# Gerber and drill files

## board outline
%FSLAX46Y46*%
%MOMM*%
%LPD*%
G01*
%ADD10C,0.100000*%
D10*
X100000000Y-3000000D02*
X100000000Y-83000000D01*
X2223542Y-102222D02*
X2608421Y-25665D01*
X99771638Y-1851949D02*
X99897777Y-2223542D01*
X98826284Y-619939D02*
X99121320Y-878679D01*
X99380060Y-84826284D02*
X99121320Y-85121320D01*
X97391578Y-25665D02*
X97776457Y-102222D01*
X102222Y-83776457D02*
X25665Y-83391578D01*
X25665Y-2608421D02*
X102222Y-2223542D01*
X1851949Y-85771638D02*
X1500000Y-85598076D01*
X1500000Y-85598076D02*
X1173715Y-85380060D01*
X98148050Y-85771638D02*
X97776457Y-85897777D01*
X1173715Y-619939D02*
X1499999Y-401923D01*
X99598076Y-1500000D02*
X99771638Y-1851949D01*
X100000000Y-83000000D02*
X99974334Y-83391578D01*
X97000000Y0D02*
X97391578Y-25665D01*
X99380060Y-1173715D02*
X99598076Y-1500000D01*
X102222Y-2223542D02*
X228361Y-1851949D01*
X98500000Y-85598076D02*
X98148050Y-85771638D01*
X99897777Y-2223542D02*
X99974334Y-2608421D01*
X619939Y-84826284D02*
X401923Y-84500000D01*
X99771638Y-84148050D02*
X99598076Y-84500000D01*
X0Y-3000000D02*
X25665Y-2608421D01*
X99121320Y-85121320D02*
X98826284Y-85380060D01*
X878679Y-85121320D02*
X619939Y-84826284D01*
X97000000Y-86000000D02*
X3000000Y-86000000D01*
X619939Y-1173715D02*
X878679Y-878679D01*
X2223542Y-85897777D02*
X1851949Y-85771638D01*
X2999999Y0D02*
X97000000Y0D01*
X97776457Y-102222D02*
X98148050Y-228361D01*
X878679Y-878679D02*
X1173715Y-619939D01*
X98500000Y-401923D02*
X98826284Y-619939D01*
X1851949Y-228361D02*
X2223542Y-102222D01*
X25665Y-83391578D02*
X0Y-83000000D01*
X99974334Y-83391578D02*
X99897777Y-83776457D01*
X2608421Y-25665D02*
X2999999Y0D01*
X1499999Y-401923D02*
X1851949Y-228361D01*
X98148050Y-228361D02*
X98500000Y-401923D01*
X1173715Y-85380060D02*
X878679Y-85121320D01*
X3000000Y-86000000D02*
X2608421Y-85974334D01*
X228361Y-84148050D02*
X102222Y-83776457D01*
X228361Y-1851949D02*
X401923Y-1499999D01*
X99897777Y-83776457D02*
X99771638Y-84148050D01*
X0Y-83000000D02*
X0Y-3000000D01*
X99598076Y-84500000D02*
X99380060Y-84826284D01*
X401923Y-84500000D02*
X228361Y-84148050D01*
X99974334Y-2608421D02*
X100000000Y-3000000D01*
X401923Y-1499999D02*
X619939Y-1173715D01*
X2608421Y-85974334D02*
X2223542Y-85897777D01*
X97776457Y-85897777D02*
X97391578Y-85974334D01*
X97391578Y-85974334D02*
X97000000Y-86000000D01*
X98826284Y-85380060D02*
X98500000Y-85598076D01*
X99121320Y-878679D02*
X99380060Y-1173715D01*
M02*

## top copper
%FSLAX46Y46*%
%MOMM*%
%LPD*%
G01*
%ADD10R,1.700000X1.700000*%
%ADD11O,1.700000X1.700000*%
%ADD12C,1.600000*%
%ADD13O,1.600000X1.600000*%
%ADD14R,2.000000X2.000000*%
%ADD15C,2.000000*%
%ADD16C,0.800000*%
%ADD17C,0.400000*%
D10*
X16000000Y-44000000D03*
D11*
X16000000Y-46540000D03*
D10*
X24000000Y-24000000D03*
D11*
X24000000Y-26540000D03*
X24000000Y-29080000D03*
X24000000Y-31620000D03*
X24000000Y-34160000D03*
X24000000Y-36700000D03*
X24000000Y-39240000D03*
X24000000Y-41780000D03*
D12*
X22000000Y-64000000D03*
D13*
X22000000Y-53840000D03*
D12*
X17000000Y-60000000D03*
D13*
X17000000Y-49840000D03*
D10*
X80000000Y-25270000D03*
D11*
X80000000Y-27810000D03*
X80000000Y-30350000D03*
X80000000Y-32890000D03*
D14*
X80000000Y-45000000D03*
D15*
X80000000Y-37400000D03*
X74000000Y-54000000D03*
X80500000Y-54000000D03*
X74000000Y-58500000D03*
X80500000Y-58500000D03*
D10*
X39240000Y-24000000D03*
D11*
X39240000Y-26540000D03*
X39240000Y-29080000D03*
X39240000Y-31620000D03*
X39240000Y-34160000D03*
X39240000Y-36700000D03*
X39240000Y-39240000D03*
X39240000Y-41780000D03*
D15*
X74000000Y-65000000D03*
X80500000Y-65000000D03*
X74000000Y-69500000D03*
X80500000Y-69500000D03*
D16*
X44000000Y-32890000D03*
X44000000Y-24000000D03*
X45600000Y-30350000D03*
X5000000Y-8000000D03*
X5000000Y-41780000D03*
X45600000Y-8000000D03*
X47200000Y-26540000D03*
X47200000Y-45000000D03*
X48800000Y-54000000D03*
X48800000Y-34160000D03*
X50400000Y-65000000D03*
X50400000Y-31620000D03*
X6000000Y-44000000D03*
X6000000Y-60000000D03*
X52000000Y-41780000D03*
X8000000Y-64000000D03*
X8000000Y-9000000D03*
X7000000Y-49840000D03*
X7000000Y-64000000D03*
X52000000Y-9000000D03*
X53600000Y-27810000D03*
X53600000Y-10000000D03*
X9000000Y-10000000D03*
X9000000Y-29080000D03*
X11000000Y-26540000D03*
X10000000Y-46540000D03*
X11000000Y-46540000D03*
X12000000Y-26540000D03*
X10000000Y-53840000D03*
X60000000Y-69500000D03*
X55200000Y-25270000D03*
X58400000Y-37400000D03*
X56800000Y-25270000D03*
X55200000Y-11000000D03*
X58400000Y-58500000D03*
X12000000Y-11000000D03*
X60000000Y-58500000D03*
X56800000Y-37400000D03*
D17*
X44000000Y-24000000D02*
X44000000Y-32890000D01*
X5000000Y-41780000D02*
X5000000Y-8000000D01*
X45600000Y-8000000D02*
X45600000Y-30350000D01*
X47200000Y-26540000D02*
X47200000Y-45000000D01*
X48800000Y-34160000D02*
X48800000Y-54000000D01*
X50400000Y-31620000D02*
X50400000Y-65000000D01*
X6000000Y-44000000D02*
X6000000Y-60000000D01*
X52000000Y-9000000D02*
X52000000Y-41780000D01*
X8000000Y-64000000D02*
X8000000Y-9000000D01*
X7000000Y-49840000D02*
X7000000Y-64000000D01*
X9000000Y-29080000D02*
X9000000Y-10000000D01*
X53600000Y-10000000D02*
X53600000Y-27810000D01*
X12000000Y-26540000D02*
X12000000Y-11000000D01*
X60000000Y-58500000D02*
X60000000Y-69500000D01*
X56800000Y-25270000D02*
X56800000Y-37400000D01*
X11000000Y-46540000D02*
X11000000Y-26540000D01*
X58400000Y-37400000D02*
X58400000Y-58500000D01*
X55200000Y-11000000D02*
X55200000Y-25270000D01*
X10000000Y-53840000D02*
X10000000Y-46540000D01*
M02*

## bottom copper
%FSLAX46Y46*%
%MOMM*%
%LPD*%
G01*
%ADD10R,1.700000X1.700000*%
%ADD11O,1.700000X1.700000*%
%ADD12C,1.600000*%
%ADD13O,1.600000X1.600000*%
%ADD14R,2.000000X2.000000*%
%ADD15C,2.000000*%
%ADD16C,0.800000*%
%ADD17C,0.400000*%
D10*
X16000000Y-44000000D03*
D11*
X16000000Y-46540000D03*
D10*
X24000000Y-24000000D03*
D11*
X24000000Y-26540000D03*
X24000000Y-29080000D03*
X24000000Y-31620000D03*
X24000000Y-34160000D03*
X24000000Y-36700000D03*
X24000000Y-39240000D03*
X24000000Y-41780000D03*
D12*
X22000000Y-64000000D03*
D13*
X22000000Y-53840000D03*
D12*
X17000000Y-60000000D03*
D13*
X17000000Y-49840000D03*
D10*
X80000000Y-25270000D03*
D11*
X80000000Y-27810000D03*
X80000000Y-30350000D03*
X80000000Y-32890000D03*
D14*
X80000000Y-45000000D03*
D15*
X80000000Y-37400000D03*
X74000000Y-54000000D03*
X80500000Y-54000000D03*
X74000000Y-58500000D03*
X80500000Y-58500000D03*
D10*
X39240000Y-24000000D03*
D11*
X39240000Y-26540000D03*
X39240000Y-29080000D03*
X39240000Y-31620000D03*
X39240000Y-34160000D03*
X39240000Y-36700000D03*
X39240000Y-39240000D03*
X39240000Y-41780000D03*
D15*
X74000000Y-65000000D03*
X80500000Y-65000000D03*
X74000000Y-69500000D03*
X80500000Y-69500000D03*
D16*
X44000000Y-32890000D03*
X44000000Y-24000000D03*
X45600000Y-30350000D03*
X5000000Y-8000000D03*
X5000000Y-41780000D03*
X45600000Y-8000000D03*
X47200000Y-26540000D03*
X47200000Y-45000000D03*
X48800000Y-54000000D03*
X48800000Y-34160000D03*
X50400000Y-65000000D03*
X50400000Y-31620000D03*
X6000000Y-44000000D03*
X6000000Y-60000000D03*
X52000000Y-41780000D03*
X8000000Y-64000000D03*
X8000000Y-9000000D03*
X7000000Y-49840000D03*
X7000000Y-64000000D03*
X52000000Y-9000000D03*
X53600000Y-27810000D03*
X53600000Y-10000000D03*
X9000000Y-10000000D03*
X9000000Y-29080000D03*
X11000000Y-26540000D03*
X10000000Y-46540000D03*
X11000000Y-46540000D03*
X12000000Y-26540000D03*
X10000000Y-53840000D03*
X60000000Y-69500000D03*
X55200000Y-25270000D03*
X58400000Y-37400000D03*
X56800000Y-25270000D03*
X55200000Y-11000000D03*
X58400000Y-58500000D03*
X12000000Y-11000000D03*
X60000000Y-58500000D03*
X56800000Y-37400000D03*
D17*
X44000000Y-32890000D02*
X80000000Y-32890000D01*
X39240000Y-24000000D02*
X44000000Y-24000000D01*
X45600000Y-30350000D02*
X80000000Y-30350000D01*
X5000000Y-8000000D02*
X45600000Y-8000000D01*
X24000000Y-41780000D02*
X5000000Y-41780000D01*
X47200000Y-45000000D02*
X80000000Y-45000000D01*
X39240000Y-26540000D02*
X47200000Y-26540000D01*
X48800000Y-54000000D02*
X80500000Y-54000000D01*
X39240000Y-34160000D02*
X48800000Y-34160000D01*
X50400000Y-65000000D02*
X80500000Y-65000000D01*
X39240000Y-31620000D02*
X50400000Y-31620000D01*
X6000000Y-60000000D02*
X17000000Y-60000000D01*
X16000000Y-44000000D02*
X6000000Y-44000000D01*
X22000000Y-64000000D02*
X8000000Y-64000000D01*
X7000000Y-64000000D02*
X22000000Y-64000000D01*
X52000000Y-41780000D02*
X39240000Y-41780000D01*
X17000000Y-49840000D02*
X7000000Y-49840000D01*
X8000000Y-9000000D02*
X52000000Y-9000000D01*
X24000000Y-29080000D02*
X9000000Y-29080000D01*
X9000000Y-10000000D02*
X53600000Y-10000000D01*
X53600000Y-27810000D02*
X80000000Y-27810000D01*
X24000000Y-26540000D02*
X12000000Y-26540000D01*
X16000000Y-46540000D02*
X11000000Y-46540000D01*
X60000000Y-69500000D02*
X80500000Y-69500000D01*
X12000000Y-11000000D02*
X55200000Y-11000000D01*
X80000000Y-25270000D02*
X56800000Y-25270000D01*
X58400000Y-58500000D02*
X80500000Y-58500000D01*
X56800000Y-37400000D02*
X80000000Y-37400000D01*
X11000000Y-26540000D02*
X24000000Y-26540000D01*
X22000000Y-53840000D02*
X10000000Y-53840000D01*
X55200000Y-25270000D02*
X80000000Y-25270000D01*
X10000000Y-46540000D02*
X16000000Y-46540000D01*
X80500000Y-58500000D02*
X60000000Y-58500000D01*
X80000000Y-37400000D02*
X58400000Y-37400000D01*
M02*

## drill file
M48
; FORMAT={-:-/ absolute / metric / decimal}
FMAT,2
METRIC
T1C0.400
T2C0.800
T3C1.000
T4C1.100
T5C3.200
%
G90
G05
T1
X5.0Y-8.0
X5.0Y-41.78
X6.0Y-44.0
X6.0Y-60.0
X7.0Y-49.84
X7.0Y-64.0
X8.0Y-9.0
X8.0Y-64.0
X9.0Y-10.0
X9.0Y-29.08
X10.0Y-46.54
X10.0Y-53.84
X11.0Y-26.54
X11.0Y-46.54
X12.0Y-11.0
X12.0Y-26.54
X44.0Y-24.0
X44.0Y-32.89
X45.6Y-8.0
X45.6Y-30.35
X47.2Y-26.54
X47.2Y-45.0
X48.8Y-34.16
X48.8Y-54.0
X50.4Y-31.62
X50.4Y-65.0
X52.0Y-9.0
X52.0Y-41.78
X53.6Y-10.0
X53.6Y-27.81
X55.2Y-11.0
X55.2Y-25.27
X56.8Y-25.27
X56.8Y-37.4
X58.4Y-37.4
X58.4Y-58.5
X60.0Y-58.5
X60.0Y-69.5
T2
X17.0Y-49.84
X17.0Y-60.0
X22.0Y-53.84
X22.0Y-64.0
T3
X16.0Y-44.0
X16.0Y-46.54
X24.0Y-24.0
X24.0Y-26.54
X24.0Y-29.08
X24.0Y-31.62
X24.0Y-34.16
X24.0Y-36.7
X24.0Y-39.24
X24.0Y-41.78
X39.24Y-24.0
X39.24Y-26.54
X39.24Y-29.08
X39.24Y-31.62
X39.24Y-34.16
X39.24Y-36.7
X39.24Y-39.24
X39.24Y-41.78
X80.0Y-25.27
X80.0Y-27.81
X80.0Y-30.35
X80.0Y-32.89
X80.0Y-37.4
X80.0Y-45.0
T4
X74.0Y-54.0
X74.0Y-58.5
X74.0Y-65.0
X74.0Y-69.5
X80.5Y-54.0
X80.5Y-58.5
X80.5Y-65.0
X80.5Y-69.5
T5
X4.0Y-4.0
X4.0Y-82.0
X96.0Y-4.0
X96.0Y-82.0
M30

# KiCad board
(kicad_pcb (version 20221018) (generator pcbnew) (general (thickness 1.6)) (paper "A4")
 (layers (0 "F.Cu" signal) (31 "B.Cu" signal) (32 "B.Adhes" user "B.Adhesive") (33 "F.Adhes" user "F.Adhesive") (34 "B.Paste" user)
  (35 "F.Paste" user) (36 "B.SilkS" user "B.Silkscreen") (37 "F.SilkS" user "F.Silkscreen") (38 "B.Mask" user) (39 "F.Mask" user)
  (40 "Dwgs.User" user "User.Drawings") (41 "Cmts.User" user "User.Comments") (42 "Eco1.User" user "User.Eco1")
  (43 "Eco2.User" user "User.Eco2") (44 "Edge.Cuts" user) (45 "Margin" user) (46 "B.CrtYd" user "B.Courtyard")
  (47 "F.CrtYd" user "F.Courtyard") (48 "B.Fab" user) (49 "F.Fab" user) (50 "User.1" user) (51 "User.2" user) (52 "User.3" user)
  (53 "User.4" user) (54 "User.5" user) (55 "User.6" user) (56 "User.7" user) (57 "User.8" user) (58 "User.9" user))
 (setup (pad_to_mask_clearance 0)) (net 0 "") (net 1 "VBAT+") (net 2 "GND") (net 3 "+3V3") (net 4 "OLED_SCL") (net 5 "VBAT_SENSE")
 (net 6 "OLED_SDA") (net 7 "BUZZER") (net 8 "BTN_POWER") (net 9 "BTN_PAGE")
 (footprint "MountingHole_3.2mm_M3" (layer "F.Cu") (at 96 4)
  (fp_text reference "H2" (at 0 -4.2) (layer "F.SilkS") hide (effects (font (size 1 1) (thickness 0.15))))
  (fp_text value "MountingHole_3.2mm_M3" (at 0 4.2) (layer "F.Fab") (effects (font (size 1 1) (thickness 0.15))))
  (pad "" np_thru_hole circle (at 0 0) (size 3.2 3.2) (drill 3.2) (layers "*.Cu" "*.Mask")))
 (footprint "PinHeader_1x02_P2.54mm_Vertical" (layer "F.Cu") (at 16 44)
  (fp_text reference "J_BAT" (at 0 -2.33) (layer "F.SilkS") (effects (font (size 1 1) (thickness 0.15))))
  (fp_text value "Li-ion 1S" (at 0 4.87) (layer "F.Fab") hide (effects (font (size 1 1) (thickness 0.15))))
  (pad "1" thru_hole rect (at 0 0) (size 1.7 1.7) (drill 1) (layers "*.Cu" "*.Mask") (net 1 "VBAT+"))
  (pad "2" thru_hole oval (at 0 2.54) (size 1.7 1.7) (drill 1) (layers "*.Cu" "*.Mask") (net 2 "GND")))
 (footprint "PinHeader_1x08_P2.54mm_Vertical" (layer "F.Cu") (at 24 24)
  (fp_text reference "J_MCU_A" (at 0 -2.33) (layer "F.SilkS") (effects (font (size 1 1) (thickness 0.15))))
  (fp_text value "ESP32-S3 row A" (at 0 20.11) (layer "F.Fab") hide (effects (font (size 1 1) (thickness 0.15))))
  (pad "1" thru_hole rect (at 0 0) (size 1.7 1.7) (drill 1) (layers "*.Cu" "*.Mask"))
  (pad "2" thru_hole oval (at 0 2.54) (size 1.7 1.7) (drill 1) (layers "*.Cu" "*.Mask") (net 2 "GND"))
  (pad "3" thru_hole oval (at 0 5.08) (size 1.7 1.7) (drill 1) (layers "*.Cu" "*.Mask") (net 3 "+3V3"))
  (pad "4" thru_hole oval (at 0 7.62) (size 1.7 1.7) (drill 1) (layers "*.Cu" "*.Mask"))
  (pad "5" thru_hole oval (at 0 10.16) (size 1.7 1.7) (drill 1) (layers "*.Cu" "*.Mask"))
  (pad "6" thru_hole oval (at 0 12.7) (size 1.7 1.7) (drill 1) (layers "*.Cu" "*.Mask"))
  (pad "7" thru_hole oval (at 0 15.24) (size 1.7 1.7) (drill 1) (layers "*.Cu" "*.Mask"))
  (pad "8" thru_hole oval (at 0 17.78) (size 1.7 1.7) (drill 1) (layers "*.Cu" "*.Mask") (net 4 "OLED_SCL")))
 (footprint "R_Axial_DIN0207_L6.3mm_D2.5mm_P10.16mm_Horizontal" (layer "F.Cu") (at 22 64 90)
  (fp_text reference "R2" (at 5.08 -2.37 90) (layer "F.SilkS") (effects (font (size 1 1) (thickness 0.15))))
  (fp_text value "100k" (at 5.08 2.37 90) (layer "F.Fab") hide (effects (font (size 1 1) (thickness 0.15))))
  (pad "1" thru_hole circle (at 0 0 90) (size 1.6 1.6) (drill 0.8) (layers "*.Cu" "*.Mask") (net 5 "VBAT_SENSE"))
  (pad "2" thru_hole oval (at 10.16 0 90) (size 1.6 1.6) (drill 0.8) (layers "*.Cu" "*.Mask") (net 2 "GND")))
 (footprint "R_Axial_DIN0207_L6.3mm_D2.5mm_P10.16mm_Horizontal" (layer "F.Cu") (at 17 60 90)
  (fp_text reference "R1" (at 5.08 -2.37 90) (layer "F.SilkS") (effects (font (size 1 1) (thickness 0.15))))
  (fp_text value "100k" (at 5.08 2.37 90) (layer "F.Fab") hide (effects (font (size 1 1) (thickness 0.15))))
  (pad "1" thru_hole circle (at 0 0 90) (size 1.6 1.6) (drill 0.8) (layers "*.Cu" "*.Mask") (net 1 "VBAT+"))
  (pad "2" thru_hole oval (at 10.16 0 90) (size 1.6 1.6) (drill 0.8) (layers "*.Cu" "*.Mask") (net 5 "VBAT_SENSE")))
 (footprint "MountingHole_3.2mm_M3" (layer "F.Cu") (at 96 82)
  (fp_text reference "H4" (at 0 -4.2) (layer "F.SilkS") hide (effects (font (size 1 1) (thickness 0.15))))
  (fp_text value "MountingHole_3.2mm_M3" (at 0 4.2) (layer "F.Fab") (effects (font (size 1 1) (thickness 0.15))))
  (pad "" np_thru_hole circle (at 0 0) (size 3.2 3.2) (drill 3.2) (layers "*.Cu" "*.Mask")))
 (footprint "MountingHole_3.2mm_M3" (layer "F.Cu") (at 4 82)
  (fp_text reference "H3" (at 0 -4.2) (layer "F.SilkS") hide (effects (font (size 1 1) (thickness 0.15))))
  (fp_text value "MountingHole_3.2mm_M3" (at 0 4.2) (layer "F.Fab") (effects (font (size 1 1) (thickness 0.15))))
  (pad "" np_thru_hole circle (at 0 0) (size 3.2 3.2) (drill 3.2) (layers "*.Cu" "*.Mask")))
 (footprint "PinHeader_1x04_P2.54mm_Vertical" (layer "F.Cu") (at 80 25.27)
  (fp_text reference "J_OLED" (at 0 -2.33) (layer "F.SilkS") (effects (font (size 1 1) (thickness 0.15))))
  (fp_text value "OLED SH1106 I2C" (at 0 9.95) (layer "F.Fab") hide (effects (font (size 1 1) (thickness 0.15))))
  (pad "1" thru_hole rect (at 0 0) (size 1.7 1.7) (drill 1) (layers "*.Cu" "*.Mask") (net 2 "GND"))
  (pad "2" thru_hole oval (at 0 2.54) (size 1.7 1.7) (drill 1) (layers "*.Cu" "*.Mask") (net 3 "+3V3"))
  (pad "3" thru_hole oval (at 0 5.08) (size 1.7 1.7) (drill 1) (layers "*.Cu" "*.Mask") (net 4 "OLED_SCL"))
  (pad "4" thru_hole oval (at 0 7.62) (size 1.7 1.7) (drill 1) (layers "*.Cu" "*.Mask") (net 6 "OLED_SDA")))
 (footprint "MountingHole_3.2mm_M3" (layer "F.Cu") (at 4 4)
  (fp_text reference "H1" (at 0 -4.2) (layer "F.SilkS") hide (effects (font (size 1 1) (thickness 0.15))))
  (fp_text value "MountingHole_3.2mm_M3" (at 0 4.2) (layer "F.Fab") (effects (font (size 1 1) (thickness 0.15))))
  (pad "" np_thru_hole circle (at 0 0) (size 3.2 3.2) (drill 3.2) (layers "*.Cu" "*.Mask")))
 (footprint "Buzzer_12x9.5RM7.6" (layer "F.Cu") (at 80 45 90)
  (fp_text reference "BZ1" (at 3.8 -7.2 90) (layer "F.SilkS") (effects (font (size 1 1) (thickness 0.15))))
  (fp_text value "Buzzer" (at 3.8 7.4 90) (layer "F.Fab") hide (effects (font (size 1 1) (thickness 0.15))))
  (pad "1" thru_hole rect (at 0 0 90) (size 2 2) (drill 1) (layers "*.Cu" "*.Mask") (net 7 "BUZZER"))
  (pad "2" thru_hole circle (at 7.6 0 90) (size 2 2) (drill 1) (layers "*.Cu" "*.Mask") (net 2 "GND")))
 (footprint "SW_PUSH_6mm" (layer "F.Cu") (at 74 54)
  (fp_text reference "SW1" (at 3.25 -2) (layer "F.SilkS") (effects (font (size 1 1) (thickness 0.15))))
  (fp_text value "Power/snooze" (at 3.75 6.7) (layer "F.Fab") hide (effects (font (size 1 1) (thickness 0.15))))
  (pad "1" thru_hole circle (at 0 0 90) (size 2 2) (drill 1.1) (layers "*.Cu" "*.Mask") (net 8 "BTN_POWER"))
  (pad "1" thru_hole circle (at 6.5 0 90) (size 2 2) (drill 1.1) (layers "*.Cu" "*.Mask") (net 8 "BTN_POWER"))
  (pad "2" thru_hole circle (at 0 4.5 90) (size 2 2) (drill 1.1) (layers "*.Cu" "*.Mask") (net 2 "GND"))
  (pad "2" thru_hole circle (at 6.5 4.5 90) (size 2 2) (drill 1.1) (layers "*.Cu" "*.Mask") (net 2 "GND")))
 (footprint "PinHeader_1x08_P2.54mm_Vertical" (layer "F.Cu") (at 39.24 24)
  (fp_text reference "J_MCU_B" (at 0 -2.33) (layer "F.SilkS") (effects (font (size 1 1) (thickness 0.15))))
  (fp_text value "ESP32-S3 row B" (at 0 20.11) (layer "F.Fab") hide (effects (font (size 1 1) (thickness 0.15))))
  (pad "1" thru_hole rect (at 0 0) (size 1.7 1.7) (drill 1) (layers "*.Cu" "*.Mask") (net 6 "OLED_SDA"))
  (pad "2" thru_hole oval (at 0 2.54) (size 1.7 1.7) (drill 1) (layers "*.Cu" "*.Mask") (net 7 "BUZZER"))
  (pad "3" thru_hole oval (at 0 5.08) (size 1.7 1.7) (drill 1) (layers "*.Cu" "*.Mask"))
  (pad "4" thru_hole oval (at 0 7.62) (size 1.7 1.7) (drill 1) (layers "*.Cu" "*.Mask") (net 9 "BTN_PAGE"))
  (pad "5" thru_hole oval (at 0 10.16) (size 1.7 1.7) (drill 1) (layers "*.Cu" "*.Mask") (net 8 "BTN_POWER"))
  (pad "6" thru_hole oval (at 0 12.7) (size 1.7 1.7) (drill 1) (layers "*.Cu" "*.Mask"))
  (pad "7" thru_hole oval (at 0 15.24) (size 1.7 1.7) (drill 1) (layers "*.Cu" "*.Mask"))
  (pad "8" thru_hole oval (at 0 17.78) (size 1.7 1.7) (drill 1) (layers "*.Cu" "*.Mask") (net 5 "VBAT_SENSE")))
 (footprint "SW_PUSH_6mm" (layer "F.Cu") (at 74 65)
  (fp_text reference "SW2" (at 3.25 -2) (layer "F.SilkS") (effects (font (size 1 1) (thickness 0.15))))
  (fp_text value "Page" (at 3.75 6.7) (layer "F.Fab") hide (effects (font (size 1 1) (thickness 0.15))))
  (pad "1" thru_hole circle (at 0 0 90) (size 2 2) (drill 1.1) (layers "*.Cu" "*.Mask") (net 9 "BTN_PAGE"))
  (pad "1" thru_hole circle (at 6.5 0 90) (size 2 2) (drill 1.1) (layers "*.Cu" "*.Mask") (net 9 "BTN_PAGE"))
  (pad "2" thru_hole circle (at 0 4.5 90) (size 2 2) (drill 1.1) (layers "*.Cu" "*.Mask") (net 2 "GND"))
  (pad "2" thru_hole circle (at 6.5 4.5 90) (size 2 2) (drill 1.1) (layers "*.Cu" "*.Mask") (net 2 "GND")))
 (gr_line (start 100 3) (end 100 83) (stroke (width 0.1) (type default)) (layer "Edge.Cuts"))
 (gr_line (start 2.223542 0.102222) (end 2.608421 0.025665) (stroke (width 0.1) (type default)) (layer "Edge.Cuts"))
 (gr_line (start 99.771638 1.851949) (end 99.897777 2.223542) (stroke (width 0.1) (type default)) (layer "Edge.Cuts"))
 (gr_line (start 98.826284 0.619939) (end 99.12132 0.878679) (stroke (width 0.1) (type default)) (layer "Edge.Cuts"))
 (gr_line (start 99.38006 84.826284) (end 99.12132 85.12132) (stroke (width 0.1) (type default)) (layer "Edge.Cuts"))
 (gr_line (start 97.391578 0.025665) (end 97.776457 0.102222) (stroke (width 0.1) (type default)) (layer "Edge.Cuts"))
 (gr_line (start 0.102222 83.776457) (end 0.025665 83.391578) (stroke (width 0.1) (type default)) (layer "Edge.Cuts"))
 (gr_line (start 0.025665 2.608421) (end 0.102222 2.223542) (stroke (width 0.1) (type default)) (layer "Edge.Cuts"))
 (gr_line (start 1.851949 85.771638) (end 1.5 85.598076) (stroke (width 0.1) (type default)) (layer "Edge.Cuts"))
 (gr_line (start 1.5 85.598076) (end 1.173715 85.38006) (stroke (width 0.1) (type default)) (layer "Edge.Cuts"))
 (gr_line (start 98.14805 85.771638) (end 97.776457 85.897777) (stroke (width 0.1) (type default)) (layer "Edge.Cuts"))
 (gr_line (start 1.173715 0.619939) (end 1.499999 0.401923) (stroke (width 0.1) (type default)) (layer "Edge.Cuts"))
 (gr_line (start 99.598076 1.5) (end 99.771638 1.851949) (stroke (width 0.1) (type default)) (layer "Edge.Cuts"))
 (gr_line (start 100 83) (end 99.974334 83.391578) (stroke (width 0.1) (type default)) (layer "Edge.Cuts"))
 (gr_line (start 97 0) (end 97.391578 0.025665) (stroke (width 0.1) (type default)) (layer "Edge.Cuts"))
 (gr_line (start 99.38006 1.173715) (end 99.598076 1.5) (stroke (width 0.1) (type default)) (layer "Edge.Cuts"))
 (gr_line (start 0.102222 2.223542) (end 0.228361 1.851949) (stroke (width 0.1) (type default)) (layer "Edge.Cuts"))
 (gr_line (start 98.5 85.598076) (end 98.14805 85.771638) (stroke (width 0.1) (type default)) (layer "Edge.Cuts"))
 (gr_line (start 99.897777 2.223542) (end 99.974334 2.608421) (stroke (width 0.1) (type default)) (layer "Edge.Cuts"))
 (gr_line (start 0.619939 84.826284) (end 0.401923 84.5) (stroke (width 0.1) (type default)) (layer "Edge.Cuts"))
 (gr_line (start 99.771638 84.14805) (end 99.598076 84.5) (stroke (width 0.1) (type default)) (layer "Edge.Cuts"))
 (gr_line (start 0 3) (end 0.025665 2.608421) (stroke (width 0.1) (type default)) (layer "Edge.Cuts"))
 (gr_line (start 99.12132 85.12132) (end 98.826284 85.38006) (stroke (width 0.1) (type default)) (layer "Edge.Cuts"))
 (gr_line (start 0.878679 85.12132) (end 0.619939 84.826284) (stroke (width 0.1) (type default)) (layer "Edge.Cuts"))
 (gr_line (start 97 86) (end 3 86) (stroke (width 0.1) (type default)) (layer "Edge.Cuts"))
 (gr_line (start 0.619939 1.173715) (end 0.878679 0.878679) (stroke (width 0.1) (type default)) (layer "Edge.Cuts"))
 (gr_line (start 2.223542 85.897777) (end 1.851949 85.771638) (stroke (width 0.1) (type default)) (layer "Edge.Cuts"))
 (gr_line (start 2.999999 0) (end 97 0) (stroke (width 0.1) (type default)) (layer "Edge.Cuts"))
 (gr_line (start 97.776457 0.102222) (end 98.14805 0.228361) (stroke (width 0.1) (type default)) (layer "Edge.Cuts"))
 (gr_line (start 0.878679 0.878679) (end 1.173715 0.619939) (stroke (width 0.1) (type default)) (layer "Edge.Cuts"))
 (gr_line (start 98.5 0.401923) (end 98.826284 0.619939) (stroke (width 0.1) (type default)) (layer "Edge.Cuts"))
 (gr_line (start 1.851949 0.228361) (end 2.223542 0.102222) (stroke (width 0.1) (type default)) (layer "Edge.Cuts"))
 (gr_line (start 0.025665 83.391578) (end 0 83) (stroke (width 0.1) (type default)) (layer "Edge.Cuts"))
 (gr_line (start 99.974334 83.391578) (end 99.897777 83.776457) (stroke (width 0.1) (type default)) (layer "Edge.Cuts"))
 (gr_line (start 2.608421 0.025665) (end 2.999999 0) (stroke (width 0.1) (type default)) (layer "Edge.Cuts"))
 (gr_line (start 1.499999 0.401923) (end 1.851949 0.228361) (stroke (width 0.1) (type default)) (layer "Edge.Cuts"))
 (gr_line (start 98.14805 0.228361) (end 98.5 0.401923) (stroke (width 0.1) (type default)) (layer "Edge.Cuts"))
 (gr_line (start 1.173715 85.38006) (end 0.878679 85.12132) (stroke (width 0.1) (type default)) (layer "Edge.Cuts"))
 (gr_line (start 3 86) (end 2.608421 85.974334) (stroke (width 0.1) (type default)) (layer "Edge.Cuts"))
 (gr_line (start 0.228361 84.14805) (end 0.102222 83.776457) (stroke (width 0.1) (type default)) (layer "Edge.Cuts"))
 (gr_line (start 0.228361 1.851949) (end 0.401923 1.499999) (stroke (width 0.1) (type default)) (layer "Edge.Cuts"))
 (gr_line (start 99.897777 83.776457) (end 99.771638 84.14805) (stroke (width 0.1) (type default)) (layer "Edge.Cuts"))
 (gr_line (start 0 83) (end 0 3) (stroke (width 0.1) (type default)) (layer "Edge.Cuts"))
 (gr_line (start 99.598076 84.5) (end 99.38006 84.826284) (stroke (width 0.1) (type default)) (layer "Edge.Cuts"))
 (gr_line (start 0.401923 84.5) (end 0.228361 84.14805) (stroke (width 0.1) (type default)) (layer "Edge.Cuts"))
 (gr_line (start 99.974334 2.608421) (end 100 3) (stroke (width 0.1) (type default)) (layer "Edge.Cuts"))
 (gr_line (start 0.401923 1.499999) (end 0.619939 1.173715) (stroke (width 0.1) (type default)) (layer "Edge.Cuts"))
 (gr_line (start 2.608421 85.974334) (end 2.223542 85.897777) (stroke (width 0.1) (type default)) (layer "Edge.Cuts"))
 (gr_line (start 97.776457 85.897777) (end 97.391578 85.974334) (stroke (width 0.1) (type default)) (layer "Edge.Cuts"))
 (gr_line (start 97.391578 85.974334) (end 97 86) (stroke (width 0.1) (type default)) (layer "Edge.Cuts"))
 (gr_line (start 98.826284 85.38006) (end 98.5 85.598076) (stroke (width 0.1) (type default)) (layer "Edge.Cuts"))
 (gr_line (start 99.12132 0.878679) (end 99.38006 1.173715) (stroke (width 0.1) (type default)) (layer "Edge.Cuts"))
 (segment (start 44 24) (end 44 32.89) (width 0.4) (layer "F.Cu") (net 6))
 (via (at 44 32.89) (size 0.8) (drill 0.4) (layers "F.Cu" "B.Cu") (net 6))
 (via (at 44 24) (size 0.8) (drill 0.4) (layers "F.Cu" "B.Cu") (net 6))
 (segment (start 44 32.89) (end 80 32.89) (width 0.4) (layer "B.Cu") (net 6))
 (segment (start 39.24 24) (end 44 24) (width 0.4) (layer "B.Cu") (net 6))
 (segment (start 5 41.78) (end 5 8) (width 0.4) (layer "F.Cu") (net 4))
 (segment (start 45.6 8) (end 45.6 30.35) (width 0.4) (layer "F.Cu") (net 4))
 (via (at 45.6 30.35) (size 0.8) (drill 0.4) (layers "F.Cu" "B.Cu") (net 4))
 (via (at 5 8) (size 0.8) (drill 0.4) (layers "F.Cu" "B.Cu") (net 4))
 (via (at 5 41.78) (size 0.8) (drill 0.4) (layers "F.Cu" "B.Cu") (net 4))
 (via (at 45.6 8) (size 0.8) (drill 0.4) (layers "F.Cu" "B.Cu") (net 4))
 (segment (start 45.6 30.35) (end 80 30.35) (width 0.4) (layer "B.Cu") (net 4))
 (segment (start 5 8) (end 45.6 8) (width 0.4) (layer "B.Cu") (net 4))
 (segment (start 24 41.78) (end 5 41.78) (width 0.4) (layer "B.Cu") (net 4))
 (segment (start 47.2 26.54) (end 47.2 45) (width 0.4) (layer "F.Cu") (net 7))
 (via (at 47.2 26.54) (size 0.8) (drill 0.4) (layers "F.Cu" "B.Cu") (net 7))
 (via (at 47.2 45) (size 0.8) (drill 0.4) (layers "F.Cu" "B.Cu") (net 7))
 (segment (start 47.2 45) (end 80 45) (width 0.4) (layer "B.Cu") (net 7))
 (segment (start 39.24 26.54) (end 47.2 26.54) (width 0.4) (layer "B.Cu") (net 7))
 (segment (start 48.8 34.16) (end 48.8 54) (width 0.4) (layer "F.Cu") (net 8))
 (via (at 48.8 54) (size 0.8) (drill 0.4) (layers "F.Cu" "B.Cu") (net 8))
 (via (at 48.8 34.16) (size 0.8) (drill 0.4) (layers "F.Cu" "B.Cu") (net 8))
 (segment (start 48.8 54) (end 80.5 54) (width 0.4) (layer "B.Cu") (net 8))
 (segment (start 39.24 34.16) (end 48.8 34.16) (width 0.4) (layer "B.Cu") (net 8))
 (segment (start 50.4 31.62) (end 50.4 65) (width 0.4) (layer "F.Cu") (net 9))
 (via (at 50.4 65) (size 0.8) (drill 0.4) (layers "F.Cu" "B.Cu") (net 9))
 (via (at 50.4 31.62) (size 0.8) (drill 0.4) (layers "F.Cu" "B.Cu") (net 9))
 (segment (start 50.4 65) (end 80.5 65) (width 0.4) (layer "B.Cu") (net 9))
 (segment (start 39.24 31.62) (end 50.4 31.62) (width 0.4) (layer "B.Cu") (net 9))
 (segment (start 6 44) (end 6 60) (width 0.4) (layer "F.Cu") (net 1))
 (via (at 6 44) (size 0.8) (drill 0.4) (layers "F.Cu" "B.Cu") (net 1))
 (via (at 6 60) (size 0.8) (drill 0.4) (layers "F.Cu" "B.Cu") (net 1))
 (segment (start 6 60) (end 17 60) (width 0.4) (layer "B.Cu") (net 1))
 (segment (start 16 44) (end 6 44) (width 0.4) (layer "B.Cu") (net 1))
 (segment (start 52 9) (end 52 41.78) (width 0.4) (layer "F.Cu") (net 5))
 (segment (start 8 64) (end 8 9) (width 0.4) (layer "F.Cu") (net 5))
 (segment (start 7 49.84) (end 7 64) (width 0.4) (layer "F.Cu") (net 5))
 (via (at 52 41.78) (size 0.8) (drill 0.4) (layers "F.Cu" "B.Cu") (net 5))
 (via (at 8 64) (size 0.8) (drill 0.4) (layers "F.Cu" "B.Cu") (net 5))
 (via (at 8 9) (size 0.8) (drill 0.4) (layers "F.Cu" "B.Cu") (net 5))
 (via (at 7 49.84) (size 0.8) (drill 0.4) (layers "F.Cu" "B.Cu") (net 5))
 (via (at 7 64) (size 0.8) (drill 0.4) (layers "F.Cu" "B.Cu") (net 5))
 (via (at 52 9) (size 0.8) (drill 0.4) (layers "F.Cu" "B.Cu") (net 5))
 (segment (start 22 64) (end 8 64) (width 0.4) (layer "B.Cu") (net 5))
 (segment (start 7 64) (end 22 64) (width 0.4) (layer "B.Cu") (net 5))
 (segment (start 52 41.78) (end 39.24 41.78) (width 0.4) (layer "B.Cu") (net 5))
 (segment (start 17 49.84) (end 7 49.84) (width 0.4) (layer "B.Cu") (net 5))
 (segment (start 8 9) (end 52 9) (width 0.4) (layer "B.Cu") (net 5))
 (segment (start 9 29.08) (end 9 10) (width 0.4) (layer "F.Cu") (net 3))
 (segment (start 53.6 10) (end 53.6 27.81) (width 0.4) (layer "F.Cu") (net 3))
 (via (at 53.6 27.81) (size 0.8) (drill 0.4) (layers "F.Cu" "B.Cu") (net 3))
 (via (at 53.6 10) (size 0.8) (drill 0.4) (layers "F.Cu" "B.Cu") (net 3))
 (via (at 9 10) (size 0.8) (drill 0.4) (layers "F.Cu" "B.Cu") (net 3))
 (via (at 9 29.08) (size 0.8) (drill 0.4) (layers "F.Cu" "B.Cu") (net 3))
 (segment (start 24 29.08) (end 9 29.08) (width 0.4) (layer "B.Cu") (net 3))
 (segment (start 9 10) (end 53.6 10) (width 0.4) (layer "B.Cu") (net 3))
 (segment (start 53.6 27.81) (end 80 27.81) (width 0.4) (layer "B.Cu") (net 3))
 (segment (start 12 26.54) (end 12 11) (width 0.4) (layer "F.Cu") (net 2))
 (segment (start 60 58.5) (end 60 69.5) (width 0.4) (layer "F.Cu") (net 2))
 (segment (start 56.8 25.27) (end 56.8 37.4) (width 0.4) (layer "F.Cu") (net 2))
 (segment (start 11 46.54) (end 11 26.54) (width 0.4) (layer "F.Cu") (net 2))
 (segment (start 58.4 37.4) (end 58.4 58.5) (width 0.4) (layer "F.Cu") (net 2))
 (segment (start 55.2 11) (end 55.2 25.27) (width 0.4) (layer "F.Cu") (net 2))
 (segment (start 10 53.84) (end 10 46.54) (width 0.4) (layer "F.Cu") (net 2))
 (via (at 11 26.54) (size 0.8) (drill 0.4) (layers "F.Cu" "B.Cu") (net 2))
 (via (at 10 46.54) (size 0.8) (drill 0.4) (layers "F.Cu" "B.Cu") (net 2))
 (via (at 11 46.54) (size 0.8) (drill 0.4) (layers "F.Cu" "B.Cu") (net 2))
 (via (at 12 26.54) (size 0.8) (drill 0.4) (layers "F.Cu" "B.Cu") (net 2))
 (via (at 10 53.84) (size 0.8) (drill 0.4) (layers "F.Cu" "B.Cu") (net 2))
 (via (at 60 69.5) (size 0.8) (drill 0.4) (layers "F.Cu" "B.Cu") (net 2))
 (via (at 55.2 25.27) (size 0.8) (drill 0.4) (layers "F.Cu" "B.Cu") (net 2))
 (via (at 58.4 37.4) (size 0.8) (drill 0.4) (layers "F.Cu" "B.Cu") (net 2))
 (via (at 56.8 25.27) (size 0.8) (drill 0.4) (layers "F.Cu" "B.Cu") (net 2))
 (via (at 55.2 11) (size 0.8) (drill 0.4) (layers "F.Cu" "B.Cu") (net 2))
 (via (at 58.4 58.5) (size 0.8) (drill 0.4) (layers "F.Cu" "B.Cu") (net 2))
 (via (at 12 11) (size 0.8) (drill 0.4) (layers "F.Cu" "B.Cu") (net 2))
 (via (at 60 58.5) (size 0.8) (drill 0.4) (layers "F.Cu" "B.Cu") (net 2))
 (via (at 56.8 37.4) (size 0.8) (drill 0.4) (layers "F.Cu" "B.Cu") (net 2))
 (segment (start 24 26.54) (end 12 26.54) (width 0.4) (layer "B.Cu") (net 2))
 (segment (start 16 46.54) (end 11 46.54) (width 0.4) (layer "B.Cu") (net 2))
 (segment (start 60 69.5) (end 80.5 69.5) (width 0.4) (layer "B.Cu") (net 2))
 (segment (start 12 11) (end 55.2 11) (width 0.4) (layer "B.Cu") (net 2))
 (segment (start 80 25.27) (end 56.8 25.27) (width 0.4) (layer "B.Cu") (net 2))
 (segment (start 58.4 58.5) (end 80.5 58.5) (width 0.4) (layer "B.Cu") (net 2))
 (segment (start 56.8 37.4) (end 80 37.4) (width 0.4) (layer "B.Cu") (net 2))
 (segment (start 11 26.54) (end 24 26.54) (width 0.4) (layer "B.Cu") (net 2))
 (segment (start 22 53.84) (end 10 53.84) (width 0.4) (layer "B.Cu") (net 2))
 (segment (start 55.2 25.27) (end 80 25.27) (width 0.4) (layer "B.Cu") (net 2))
 (segment (start 10 46.54) (end 16 46.54) (width 0.4) (layer "B.Cu") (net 2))
 (segment (start 80.5 58.5) (end 60 58.5) (width 0.4) (layer "B.Cu") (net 2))
 (segment (start 80 37.4) (end 58.4 37.4) (width 0.4) (layer "B.Cu") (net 2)))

